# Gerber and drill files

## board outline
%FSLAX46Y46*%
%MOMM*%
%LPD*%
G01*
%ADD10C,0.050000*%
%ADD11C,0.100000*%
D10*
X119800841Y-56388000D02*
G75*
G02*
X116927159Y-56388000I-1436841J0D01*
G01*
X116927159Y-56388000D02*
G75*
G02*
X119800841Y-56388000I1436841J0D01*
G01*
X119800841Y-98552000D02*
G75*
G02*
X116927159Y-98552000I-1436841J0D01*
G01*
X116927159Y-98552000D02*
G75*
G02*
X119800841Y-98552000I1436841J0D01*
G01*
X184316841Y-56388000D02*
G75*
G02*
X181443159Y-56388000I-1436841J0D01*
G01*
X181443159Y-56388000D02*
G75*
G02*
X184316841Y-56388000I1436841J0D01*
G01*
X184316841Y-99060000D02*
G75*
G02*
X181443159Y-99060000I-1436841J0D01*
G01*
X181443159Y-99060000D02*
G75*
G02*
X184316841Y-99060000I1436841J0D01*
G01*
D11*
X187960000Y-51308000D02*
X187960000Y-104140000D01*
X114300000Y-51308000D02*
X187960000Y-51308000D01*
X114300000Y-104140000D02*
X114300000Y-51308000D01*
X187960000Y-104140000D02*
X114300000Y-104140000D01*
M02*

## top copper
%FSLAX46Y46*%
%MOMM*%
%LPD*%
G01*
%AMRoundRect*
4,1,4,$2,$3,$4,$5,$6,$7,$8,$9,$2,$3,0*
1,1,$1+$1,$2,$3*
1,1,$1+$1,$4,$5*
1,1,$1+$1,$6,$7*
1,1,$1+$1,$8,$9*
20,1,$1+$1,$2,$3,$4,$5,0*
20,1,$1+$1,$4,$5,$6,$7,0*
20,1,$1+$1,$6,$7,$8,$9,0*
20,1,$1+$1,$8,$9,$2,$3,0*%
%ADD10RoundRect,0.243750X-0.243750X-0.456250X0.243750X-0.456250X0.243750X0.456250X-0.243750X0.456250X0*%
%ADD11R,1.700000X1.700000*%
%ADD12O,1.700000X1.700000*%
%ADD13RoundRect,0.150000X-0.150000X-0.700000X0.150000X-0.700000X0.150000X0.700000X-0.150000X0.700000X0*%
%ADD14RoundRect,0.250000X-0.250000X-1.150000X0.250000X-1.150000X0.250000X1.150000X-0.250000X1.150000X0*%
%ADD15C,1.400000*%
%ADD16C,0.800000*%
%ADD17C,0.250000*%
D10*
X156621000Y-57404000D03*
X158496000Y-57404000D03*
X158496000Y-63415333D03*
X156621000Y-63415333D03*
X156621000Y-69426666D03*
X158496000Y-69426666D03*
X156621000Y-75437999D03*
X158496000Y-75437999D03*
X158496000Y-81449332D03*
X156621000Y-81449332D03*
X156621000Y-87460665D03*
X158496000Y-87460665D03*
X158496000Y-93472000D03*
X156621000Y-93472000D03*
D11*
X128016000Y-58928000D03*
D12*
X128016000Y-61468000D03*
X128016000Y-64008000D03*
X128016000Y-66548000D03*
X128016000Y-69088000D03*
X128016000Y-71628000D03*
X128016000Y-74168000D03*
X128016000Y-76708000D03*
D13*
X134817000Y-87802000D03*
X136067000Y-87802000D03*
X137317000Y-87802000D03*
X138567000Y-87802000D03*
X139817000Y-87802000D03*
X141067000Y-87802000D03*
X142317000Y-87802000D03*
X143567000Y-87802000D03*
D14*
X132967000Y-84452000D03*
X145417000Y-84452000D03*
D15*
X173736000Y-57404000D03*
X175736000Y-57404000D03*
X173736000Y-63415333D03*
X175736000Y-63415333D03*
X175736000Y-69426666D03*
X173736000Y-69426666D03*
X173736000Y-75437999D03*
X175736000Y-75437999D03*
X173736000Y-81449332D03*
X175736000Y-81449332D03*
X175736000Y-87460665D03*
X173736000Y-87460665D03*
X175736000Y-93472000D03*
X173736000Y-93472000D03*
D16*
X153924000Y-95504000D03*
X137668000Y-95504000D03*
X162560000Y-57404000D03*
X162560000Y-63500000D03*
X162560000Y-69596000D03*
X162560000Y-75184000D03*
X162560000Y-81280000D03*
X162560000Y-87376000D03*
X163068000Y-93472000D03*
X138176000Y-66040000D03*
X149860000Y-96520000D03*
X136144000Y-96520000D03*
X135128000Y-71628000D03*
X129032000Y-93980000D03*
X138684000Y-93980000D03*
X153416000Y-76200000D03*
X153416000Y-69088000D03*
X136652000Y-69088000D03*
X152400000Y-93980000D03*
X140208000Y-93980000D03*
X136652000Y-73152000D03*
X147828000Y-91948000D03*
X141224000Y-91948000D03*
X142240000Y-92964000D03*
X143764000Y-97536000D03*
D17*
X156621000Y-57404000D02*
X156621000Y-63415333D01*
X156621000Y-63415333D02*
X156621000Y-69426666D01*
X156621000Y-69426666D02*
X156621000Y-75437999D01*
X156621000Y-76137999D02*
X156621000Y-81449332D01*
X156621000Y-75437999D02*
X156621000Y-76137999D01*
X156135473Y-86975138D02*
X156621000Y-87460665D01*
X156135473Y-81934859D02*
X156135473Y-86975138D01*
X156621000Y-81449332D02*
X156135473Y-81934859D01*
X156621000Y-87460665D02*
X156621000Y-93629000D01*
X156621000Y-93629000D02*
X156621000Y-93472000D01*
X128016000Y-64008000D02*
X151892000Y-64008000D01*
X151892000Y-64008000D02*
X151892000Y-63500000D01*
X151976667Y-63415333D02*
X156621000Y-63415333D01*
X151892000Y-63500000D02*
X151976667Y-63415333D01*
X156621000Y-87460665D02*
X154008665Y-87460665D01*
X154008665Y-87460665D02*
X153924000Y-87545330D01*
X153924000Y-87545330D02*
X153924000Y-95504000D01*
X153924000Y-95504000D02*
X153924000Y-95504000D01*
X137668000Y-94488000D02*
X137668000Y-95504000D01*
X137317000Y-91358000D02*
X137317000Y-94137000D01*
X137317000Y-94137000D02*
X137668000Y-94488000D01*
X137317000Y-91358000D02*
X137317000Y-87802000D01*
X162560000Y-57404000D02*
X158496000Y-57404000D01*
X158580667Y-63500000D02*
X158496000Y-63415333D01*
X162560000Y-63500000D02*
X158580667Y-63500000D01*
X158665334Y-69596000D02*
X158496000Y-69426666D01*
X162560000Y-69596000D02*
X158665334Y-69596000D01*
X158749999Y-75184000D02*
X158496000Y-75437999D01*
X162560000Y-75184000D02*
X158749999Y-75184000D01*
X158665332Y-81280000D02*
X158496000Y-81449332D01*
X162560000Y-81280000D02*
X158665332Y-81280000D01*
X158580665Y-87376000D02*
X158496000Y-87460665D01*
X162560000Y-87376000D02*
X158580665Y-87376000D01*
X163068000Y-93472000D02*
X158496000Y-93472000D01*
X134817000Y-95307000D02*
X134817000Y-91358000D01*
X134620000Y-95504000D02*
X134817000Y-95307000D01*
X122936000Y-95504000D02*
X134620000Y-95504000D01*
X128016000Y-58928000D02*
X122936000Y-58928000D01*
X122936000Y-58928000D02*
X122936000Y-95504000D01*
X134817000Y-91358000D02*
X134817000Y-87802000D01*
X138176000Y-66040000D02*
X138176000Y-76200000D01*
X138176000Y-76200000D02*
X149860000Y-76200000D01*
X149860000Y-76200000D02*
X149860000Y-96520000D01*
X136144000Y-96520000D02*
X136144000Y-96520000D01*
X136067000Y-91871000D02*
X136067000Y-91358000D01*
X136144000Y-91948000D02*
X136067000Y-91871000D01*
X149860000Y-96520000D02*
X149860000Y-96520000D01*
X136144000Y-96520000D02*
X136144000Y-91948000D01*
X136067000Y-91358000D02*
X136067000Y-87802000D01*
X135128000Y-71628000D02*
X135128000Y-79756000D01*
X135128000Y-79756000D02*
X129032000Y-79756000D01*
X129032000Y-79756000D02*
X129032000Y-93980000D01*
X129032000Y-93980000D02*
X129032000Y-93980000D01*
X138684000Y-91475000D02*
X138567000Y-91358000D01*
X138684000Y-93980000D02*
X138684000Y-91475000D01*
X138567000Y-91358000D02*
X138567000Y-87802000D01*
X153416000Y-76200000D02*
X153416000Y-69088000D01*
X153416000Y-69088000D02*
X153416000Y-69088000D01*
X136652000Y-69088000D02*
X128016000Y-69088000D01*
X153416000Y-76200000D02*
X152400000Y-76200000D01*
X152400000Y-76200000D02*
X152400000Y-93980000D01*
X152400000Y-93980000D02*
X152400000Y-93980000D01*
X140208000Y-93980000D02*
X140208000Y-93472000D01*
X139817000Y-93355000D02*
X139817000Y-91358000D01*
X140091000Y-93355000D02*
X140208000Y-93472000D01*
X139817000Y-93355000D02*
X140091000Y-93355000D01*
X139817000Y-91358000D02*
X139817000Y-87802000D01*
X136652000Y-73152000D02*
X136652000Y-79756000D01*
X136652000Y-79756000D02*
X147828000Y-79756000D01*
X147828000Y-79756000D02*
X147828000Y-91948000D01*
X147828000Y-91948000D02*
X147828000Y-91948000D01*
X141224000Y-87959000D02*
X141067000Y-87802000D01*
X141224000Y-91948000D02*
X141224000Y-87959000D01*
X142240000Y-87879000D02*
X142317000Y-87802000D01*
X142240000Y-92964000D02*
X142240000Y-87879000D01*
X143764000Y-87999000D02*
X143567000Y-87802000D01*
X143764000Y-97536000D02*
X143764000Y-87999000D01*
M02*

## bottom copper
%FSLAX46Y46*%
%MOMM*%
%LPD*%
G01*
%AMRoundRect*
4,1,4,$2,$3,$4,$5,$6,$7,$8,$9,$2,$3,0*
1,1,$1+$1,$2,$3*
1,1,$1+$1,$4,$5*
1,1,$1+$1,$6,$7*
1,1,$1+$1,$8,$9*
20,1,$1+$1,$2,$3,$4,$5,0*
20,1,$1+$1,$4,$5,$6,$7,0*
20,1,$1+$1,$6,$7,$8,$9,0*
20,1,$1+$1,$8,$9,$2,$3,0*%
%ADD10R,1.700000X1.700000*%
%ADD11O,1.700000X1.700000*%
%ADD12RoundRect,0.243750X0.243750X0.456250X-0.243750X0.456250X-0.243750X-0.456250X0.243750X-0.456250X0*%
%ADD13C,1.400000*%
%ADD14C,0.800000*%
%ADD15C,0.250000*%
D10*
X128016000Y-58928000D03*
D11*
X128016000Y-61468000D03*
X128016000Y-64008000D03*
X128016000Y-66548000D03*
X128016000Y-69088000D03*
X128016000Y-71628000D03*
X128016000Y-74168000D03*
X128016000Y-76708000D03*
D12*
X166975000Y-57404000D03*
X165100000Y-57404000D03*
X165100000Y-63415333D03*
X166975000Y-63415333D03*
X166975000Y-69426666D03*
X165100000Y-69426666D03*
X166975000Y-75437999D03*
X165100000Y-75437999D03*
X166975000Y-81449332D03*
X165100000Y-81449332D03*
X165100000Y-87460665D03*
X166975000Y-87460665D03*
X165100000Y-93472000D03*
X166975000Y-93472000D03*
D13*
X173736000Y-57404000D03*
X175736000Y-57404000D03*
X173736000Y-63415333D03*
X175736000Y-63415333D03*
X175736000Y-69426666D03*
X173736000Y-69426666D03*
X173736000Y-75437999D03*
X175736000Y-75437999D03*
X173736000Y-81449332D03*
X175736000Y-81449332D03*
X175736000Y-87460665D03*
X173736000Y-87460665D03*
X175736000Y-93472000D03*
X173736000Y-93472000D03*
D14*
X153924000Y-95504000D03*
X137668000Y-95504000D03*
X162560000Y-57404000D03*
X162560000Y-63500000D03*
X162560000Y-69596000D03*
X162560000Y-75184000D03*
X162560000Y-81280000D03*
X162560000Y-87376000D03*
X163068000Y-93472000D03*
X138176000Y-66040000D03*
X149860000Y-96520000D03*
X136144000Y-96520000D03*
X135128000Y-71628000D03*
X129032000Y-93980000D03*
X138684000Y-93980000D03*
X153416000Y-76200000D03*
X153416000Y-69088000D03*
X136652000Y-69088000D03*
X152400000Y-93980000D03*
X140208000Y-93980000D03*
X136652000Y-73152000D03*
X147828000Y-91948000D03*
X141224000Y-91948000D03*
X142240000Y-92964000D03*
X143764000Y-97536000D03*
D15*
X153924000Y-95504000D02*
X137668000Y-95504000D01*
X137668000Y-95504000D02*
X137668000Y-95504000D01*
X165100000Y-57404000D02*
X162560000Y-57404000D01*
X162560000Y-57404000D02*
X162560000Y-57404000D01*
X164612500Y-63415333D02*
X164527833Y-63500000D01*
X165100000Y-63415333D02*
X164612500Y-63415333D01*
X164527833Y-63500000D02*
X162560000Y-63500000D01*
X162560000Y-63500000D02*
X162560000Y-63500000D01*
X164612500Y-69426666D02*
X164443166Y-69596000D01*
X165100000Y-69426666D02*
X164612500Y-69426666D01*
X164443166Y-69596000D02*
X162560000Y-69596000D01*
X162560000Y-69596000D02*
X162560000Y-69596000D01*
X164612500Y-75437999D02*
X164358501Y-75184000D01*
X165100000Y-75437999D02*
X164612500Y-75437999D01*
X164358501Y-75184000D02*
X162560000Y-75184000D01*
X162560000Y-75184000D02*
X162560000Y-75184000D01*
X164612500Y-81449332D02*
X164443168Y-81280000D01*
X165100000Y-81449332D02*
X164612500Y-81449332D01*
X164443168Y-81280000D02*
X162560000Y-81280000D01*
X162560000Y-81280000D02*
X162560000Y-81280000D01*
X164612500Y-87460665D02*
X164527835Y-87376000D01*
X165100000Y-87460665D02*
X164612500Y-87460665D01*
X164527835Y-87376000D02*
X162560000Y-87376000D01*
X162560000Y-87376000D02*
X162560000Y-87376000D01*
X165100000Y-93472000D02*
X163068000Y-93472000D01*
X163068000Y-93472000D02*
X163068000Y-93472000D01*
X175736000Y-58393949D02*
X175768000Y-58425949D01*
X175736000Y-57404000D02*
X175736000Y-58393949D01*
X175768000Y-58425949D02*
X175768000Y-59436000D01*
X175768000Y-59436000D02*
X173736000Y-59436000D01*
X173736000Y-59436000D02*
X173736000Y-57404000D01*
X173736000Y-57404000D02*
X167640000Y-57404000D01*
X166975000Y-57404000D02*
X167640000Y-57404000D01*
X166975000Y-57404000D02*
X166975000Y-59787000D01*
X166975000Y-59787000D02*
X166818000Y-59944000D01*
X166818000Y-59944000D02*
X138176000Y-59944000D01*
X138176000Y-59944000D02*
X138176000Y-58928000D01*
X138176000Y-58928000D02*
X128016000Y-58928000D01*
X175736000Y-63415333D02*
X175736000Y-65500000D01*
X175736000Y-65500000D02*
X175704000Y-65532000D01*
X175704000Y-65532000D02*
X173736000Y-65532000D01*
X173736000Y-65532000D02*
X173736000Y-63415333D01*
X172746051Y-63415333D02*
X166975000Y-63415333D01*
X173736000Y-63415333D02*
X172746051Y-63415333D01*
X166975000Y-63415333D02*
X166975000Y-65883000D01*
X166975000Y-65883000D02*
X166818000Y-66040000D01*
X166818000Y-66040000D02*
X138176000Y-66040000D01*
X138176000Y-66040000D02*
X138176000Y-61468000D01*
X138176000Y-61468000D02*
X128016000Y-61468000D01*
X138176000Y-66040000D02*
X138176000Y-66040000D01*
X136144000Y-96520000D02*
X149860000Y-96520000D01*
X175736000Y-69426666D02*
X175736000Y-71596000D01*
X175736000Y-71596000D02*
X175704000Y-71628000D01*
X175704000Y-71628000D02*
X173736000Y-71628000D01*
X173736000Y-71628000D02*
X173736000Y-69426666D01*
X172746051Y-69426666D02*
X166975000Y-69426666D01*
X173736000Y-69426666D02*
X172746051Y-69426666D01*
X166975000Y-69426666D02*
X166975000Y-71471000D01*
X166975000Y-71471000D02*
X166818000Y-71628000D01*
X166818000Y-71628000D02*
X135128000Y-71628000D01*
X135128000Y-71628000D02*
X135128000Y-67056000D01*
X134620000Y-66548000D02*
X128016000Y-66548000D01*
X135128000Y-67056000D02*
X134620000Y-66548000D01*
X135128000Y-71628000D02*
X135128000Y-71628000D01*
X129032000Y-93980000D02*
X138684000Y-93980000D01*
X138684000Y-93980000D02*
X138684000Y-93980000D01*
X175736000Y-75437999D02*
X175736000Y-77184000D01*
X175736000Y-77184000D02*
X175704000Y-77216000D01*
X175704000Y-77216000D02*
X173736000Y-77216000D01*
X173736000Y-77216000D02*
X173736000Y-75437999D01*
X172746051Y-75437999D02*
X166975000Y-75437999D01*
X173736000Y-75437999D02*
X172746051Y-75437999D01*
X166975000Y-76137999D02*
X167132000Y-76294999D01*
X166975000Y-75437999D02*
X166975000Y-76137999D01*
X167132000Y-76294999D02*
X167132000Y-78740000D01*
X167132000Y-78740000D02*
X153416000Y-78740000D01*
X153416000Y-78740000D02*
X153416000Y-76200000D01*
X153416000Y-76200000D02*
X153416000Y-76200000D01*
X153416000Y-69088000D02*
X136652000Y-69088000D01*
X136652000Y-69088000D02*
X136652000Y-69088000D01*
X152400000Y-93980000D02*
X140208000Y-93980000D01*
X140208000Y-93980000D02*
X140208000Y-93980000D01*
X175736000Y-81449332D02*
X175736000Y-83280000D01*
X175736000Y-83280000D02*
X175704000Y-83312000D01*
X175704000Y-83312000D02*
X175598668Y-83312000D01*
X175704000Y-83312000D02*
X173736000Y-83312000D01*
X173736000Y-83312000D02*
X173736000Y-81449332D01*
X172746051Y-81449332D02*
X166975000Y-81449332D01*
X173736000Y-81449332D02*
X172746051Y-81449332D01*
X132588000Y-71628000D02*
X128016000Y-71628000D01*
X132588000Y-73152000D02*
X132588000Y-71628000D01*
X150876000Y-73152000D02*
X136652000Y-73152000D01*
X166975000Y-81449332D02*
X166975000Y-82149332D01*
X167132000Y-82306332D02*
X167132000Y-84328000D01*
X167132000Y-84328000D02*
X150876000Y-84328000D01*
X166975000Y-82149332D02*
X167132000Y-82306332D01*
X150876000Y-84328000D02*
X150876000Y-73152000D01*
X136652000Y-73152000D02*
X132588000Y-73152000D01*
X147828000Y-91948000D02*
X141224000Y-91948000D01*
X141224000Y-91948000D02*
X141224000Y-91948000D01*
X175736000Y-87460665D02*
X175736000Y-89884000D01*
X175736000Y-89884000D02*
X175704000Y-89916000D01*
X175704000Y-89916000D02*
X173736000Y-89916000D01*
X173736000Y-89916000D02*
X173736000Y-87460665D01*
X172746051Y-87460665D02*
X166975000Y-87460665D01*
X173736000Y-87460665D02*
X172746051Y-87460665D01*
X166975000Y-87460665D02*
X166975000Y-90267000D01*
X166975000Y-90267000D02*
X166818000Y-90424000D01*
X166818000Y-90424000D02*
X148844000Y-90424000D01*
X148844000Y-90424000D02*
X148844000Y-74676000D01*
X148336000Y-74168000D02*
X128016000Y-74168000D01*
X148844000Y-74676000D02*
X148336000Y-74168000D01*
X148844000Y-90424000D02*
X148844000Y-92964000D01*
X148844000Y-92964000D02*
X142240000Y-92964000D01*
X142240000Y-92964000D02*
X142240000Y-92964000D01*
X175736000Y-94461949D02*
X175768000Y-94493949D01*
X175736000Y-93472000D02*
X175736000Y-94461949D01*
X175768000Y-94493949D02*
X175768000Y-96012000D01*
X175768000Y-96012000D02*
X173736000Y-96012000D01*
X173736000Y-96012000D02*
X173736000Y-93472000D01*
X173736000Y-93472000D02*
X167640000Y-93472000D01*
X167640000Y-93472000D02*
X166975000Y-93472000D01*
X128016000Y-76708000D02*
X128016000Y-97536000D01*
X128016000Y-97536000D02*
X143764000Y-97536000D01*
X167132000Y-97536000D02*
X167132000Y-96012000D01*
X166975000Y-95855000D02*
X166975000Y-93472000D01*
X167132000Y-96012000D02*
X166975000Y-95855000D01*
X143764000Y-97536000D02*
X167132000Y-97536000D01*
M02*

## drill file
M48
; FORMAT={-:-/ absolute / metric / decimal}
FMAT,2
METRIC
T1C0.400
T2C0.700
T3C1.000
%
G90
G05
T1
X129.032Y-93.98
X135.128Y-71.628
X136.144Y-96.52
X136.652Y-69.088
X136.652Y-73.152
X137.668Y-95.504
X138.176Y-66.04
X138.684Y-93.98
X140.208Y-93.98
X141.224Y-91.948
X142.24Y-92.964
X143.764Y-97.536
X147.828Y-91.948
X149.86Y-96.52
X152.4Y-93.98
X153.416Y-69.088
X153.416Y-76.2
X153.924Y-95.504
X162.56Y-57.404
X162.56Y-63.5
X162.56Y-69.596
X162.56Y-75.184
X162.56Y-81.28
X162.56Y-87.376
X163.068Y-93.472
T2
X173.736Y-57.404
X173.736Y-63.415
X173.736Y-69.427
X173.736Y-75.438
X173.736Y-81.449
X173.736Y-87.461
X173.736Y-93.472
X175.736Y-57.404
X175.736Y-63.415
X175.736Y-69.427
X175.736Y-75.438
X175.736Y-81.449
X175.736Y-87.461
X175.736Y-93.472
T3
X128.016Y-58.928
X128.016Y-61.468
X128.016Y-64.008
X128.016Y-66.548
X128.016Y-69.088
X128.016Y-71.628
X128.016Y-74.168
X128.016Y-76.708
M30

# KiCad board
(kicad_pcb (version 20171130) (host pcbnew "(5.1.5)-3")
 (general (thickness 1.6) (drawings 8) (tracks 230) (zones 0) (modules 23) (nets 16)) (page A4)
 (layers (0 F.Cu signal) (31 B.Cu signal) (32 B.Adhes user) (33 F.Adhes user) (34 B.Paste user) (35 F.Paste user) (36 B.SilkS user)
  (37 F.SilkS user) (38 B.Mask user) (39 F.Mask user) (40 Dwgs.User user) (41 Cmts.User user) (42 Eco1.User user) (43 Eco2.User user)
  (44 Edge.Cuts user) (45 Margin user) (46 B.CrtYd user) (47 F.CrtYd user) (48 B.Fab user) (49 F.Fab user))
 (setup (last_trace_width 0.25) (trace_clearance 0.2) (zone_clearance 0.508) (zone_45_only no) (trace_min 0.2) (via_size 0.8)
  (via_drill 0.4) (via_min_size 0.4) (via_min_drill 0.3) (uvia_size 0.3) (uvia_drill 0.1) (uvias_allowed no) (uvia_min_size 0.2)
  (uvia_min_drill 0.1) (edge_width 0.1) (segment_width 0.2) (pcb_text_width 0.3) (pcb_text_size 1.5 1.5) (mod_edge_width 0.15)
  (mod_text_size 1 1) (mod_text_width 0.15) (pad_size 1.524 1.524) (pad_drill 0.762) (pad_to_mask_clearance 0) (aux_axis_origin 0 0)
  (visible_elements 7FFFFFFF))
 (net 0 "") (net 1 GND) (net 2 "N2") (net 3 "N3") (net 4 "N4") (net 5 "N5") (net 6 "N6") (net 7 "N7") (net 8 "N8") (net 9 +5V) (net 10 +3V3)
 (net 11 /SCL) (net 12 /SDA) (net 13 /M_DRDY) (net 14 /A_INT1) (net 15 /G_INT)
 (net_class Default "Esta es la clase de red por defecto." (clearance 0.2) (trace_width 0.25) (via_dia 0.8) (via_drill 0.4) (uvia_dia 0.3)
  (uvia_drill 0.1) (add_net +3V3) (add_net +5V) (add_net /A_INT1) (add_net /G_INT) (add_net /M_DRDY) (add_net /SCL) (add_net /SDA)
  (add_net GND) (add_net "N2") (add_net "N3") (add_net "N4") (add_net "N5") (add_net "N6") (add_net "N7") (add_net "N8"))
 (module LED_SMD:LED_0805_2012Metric (layer F.Cu) (at 157.5585 57.404)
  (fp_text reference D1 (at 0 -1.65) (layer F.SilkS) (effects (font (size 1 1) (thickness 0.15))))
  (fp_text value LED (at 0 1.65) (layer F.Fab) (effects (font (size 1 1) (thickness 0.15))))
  (pad 1 smd roundrect (at -0.9375 0) (size 0.975 1.4) (layers F.Cu F.Paste F.Mask) (roundrect_rratio 0.25) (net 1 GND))
  (pad 2 smd roundrect (at 0.9375 0) (size 0.975 1.4) (layers F.Cu F.Paste F.Mask) (roundrect_rratio 0.25) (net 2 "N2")))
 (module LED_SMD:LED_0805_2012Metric (layer F.Cu) (at 157.5585 63.415333)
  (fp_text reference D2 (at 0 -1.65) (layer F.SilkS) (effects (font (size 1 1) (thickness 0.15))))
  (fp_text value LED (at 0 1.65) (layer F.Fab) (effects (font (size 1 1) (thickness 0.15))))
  (pad 2 smd roundrect (at 0.9375 0) (size 0.975 1.4) (layers F.Cu F.Paste F.Mask) (roundrect_rratio 0.25) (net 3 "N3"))
  (pad 1 smd roundrect (at -0.9375 0) (size 0.975 1.4) (layers F.Cu F.Paste F.Mask) (roundrect_rratio 0.25) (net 1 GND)))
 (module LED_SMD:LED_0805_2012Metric (layer F.Cu) (at 157.5585 69.426666)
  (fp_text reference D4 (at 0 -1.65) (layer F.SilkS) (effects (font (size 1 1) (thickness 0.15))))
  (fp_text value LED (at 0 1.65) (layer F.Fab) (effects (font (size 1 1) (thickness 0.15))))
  (pad 1 smd roundrect (at -0.9375 0) (size 0.975 1.4) (layers F.Cu F.Paste F.Mask) (roundrect_rratio 0.25) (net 1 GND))
  (pad 2 smd roundrect (at 0.9375 0) (size 0.975 1.4) (layers F.Cu F.Paste F.Mask) (roundrect_rratio 0.25) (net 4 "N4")))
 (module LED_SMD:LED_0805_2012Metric (layer F.Cu) (at 157.5585 75.437999)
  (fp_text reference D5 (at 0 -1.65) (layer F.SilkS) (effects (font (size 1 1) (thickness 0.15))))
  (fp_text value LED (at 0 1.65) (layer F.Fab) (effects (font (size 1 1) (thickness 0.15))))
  (pad 1 smd roundrect (at -0.9375 0) (size 0.975 1.4) (layers F.Cu F.Paste F.Mask) (roundrect_rratio 0.25) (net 1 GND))
  (pad 2 smd roundrect (at 0.9375 0) (size 0.975 1.4) (layers F.Cu F.Paste F.Mask) (roundrect_rratio 0.25) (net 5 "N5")))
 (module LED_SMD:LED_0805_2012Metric (layer F.Cu) (at 157.5585 81.449332)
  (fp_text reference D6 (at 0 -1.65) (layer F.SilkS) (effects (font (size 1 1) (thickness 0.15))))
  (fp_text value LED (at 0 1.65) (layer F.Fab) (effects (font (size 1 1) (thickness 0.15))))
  (pad 2 smd roundrect (at 0.9375 0) (size 0.975 1.4) (layers F.Cu F.Paste F.Mask) (roundrect_rratio 0.25) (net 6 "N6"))
  (pad 1 smd roundrect (at -0.9375 0) (size 0.975 1.4) (layers F.Cu F.Paste F.Mask) (roundrect_rratio 0.25) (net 1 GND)))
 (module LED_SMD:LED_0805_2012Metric (layer F.Cu) (at 157.5585 87.460665)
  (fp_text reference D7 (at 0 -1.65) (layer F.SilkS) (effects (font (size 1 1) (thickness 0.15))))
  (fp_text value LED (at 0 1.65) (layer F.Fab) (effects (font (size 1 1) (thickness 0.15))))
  (pad 1 smd roundrect (at -0.9375 0) (size 0.975 1.4) (layers F.Cu F.Paste F.Mask) (roundrect_rratio 0.25) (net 1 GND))
  (pad 2 smd roundrect (at 0.9375 0) (size 0.975 1.4) (layers F.Cu F.Paste F.Mask) (roundrect_rratio 0.25) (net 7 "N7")))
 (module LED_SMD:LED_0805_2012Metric (layer F.Cu) (at 157.5585 93.472)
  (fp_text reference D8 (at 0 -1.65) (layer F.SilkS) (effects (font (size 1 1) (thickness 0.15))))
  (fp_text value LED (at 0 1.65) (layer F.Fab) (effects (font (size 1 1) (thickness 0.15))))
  (pad 2 smd roundrect (at 0.9375 0) (size 0.975 1.4) (layers F.Cu F.Paste F.Mask) (roundrect_rratio 0.25) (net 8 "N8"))
  (pad 1 smd roundrect (at -0.9375 0) (size 0.975 1.4) (layers F.Cu F.Paste F.Mask) (roundrect_rratio 0.25) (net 1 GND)))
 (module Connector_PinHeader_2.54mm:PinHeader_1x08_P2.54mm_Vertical (layer F.Cu) (at 128.016 58.928)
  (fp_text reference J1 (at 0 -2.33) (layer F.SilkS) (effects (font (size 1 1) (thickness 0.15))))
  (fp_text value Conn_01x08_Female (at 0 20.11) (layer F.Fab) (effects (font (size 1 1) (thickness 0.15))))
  (pad 1 thru_hole rect (at 0 0) (size 1.7 1.7) (drill 1) (layers *.Cu *.Mask) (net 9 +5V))
  (pad 2 thru_hole oval (at 0 2.54) (size 1.7 1.7) (drill 1) (layers *.Cu *.Mask) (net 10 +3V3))
  (pad 3 thru_hole oval (at 0 5.08) (size 1.7 1.7) (drill 1) (layers *.Cu *.Mask) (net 1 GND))
  (pad 4 thru_hole oval (at 0 7.62) (size 1.7 1.7) (drill 1) (layers *.Cu *.Mask) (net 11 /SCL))
  (pad 5 thru_hole oval (at 0 10.16) (size 1.7 1.7) (drill 1) (layers *.Cu *.Mask) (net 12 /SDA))
  (pad 6 thru_hole oval (at 0 12.7) (size 1.7 1.7) (drill 1) (layers *.Cu *.Mask) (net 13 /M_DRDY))
  (pad 7 thru_hole oval (at 0 15.24) (size 1.7 1.7) (drill 1) (layers *.Cu *.Mask) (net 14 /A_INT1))
  (pad 8 thru_hole oval (at 0 17.78) (size 1.7 1.7) (drill 1) (layers *.Cu *.Mask) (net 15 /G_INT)))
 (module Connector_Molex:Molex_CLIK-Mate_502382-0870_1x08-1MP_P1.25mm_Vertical (layer F.Cu) (at 139.192 85.852)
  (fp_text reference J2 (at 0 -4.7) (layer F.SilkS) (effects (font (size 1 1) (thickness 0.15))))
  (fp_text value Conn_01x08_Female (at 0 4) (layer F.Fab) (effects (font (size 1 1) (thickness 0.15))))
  (pad 1 smd roundrect (at -4.375 1.95) (size 0.6 1.7) (layers F.Cu F.Paste F.Mask) (roundrect_rratio 0.25) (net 9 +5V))
  (pad 2 smd roundrect (at -3.125 1.95) (size 0.6 1.7) (layers F.Cu F.Paste F.Mask) (roundrect_rratio 0.25) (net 10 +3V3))
  (pad 3 smd roundrect (at -1.875 1.95) (size 0.6 1.7) (layers F.Cu F.Paste F.Mask) (roundrect_rratio 0.25) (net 1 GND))
  (pad 4 smd roundrect (at -0.625 1.95) (size 0.6 1.7) (layers F.Cu F.Paste F.Mask) (roundrect_rratio 0.25) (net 11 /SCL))
  (pad 5 smd roundrect (at 0.625 1.95) (size 0.6 1.7) (layers F.Cu F.Paste F.Mask) (roundrect_rratio 0.25) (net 12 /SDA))
  (pad 6 smd roundrect (at 1.875 1.95) (size 0.6 1.7) (layers F.Cu F.Paste F.Mask) (roundrect_rratio 0.25) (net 13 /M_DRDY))
  (pad 7 smd roundrect (at 3.125 1.95) (size 0.6 1.7) (layers F.Cu F.Paste F.Mask) (roundrect_rratio 0.25) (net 14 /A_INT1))
  (pad 8 smd roundrect (at 4.375 1.95) (size 0.6 1.7) (layers F.Cu F.Paste F.Mask) (roundrect_rratio 0.25) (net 15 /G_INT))
  (pad MP smd roundrect (at -6.225 -1.4) (size 1 2.8) (layers F.Cu F.Paste F.Mask) (roundrect_rratio 0.25))
  (pad MP smd roundrect (at 6.225 -1.4) (size 1 2.8) (layers F.Cu F.Paste F.Mask) (roundrect_rratio 0.25)))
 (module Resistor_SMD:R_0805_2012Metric (layer B.Cu) (at 166.0375 57.404 180)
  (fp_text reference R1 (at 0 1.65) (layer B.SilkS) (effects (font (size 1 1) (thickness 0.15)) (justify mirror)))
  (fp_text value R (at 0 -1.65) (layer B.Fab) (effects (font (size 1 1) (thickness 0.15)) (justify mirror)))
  (pad 1 smd roundrect (at -0.9375 0 180) (size 0.975 1.4) (layers B.Cu B.Paste B.Mask) (roundrect_rratio 0.25) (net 9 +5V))
  (pad 2 smd roundrect (at 0.9375 0 180) (size 0.975 1.4) (layers B.Cu B.Paste B.Mask) (roundrect_rratio 0.25) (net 2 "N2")))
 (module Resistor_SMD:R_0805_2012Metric (layer B.Cu) (at 166.0375 63.415333 180)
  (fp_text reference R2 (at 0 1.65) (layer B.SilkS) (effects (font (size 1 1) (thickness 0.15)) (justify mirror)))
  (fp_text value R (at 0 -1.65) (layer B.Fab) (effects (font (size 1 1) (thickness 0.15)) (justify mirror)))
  (pad 2 smd roundrect (at 0.9375 0 180) (size 0.975 1.4) (layers B.Cu B.Paste B.Mask) (roundrect_rratio 0.25) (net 3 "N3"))
  (pad 1 smd roundrect (at -0.9375 0 180) (size 0.975 1.4) (layers B.Cu B.Paste B.Mask) (roundrect_rratio 0.25) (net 10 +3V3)))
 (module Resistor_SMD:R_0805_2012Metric (layer B.Cu) (at 166.0375 69.426666 180)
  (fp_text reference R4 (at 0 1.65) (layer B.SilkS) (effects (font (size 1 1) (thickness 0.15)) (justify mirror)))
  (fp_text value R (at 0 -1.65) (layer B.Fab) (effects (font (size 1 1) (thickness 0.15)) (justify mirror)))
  (pad 1 smd roundrect (at -0.9375 0 180) (size 0.975 1.4) (layers B.Cu B.Paste B.Mask) (roundrect_rratio 0.25) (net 11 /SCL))
  (pad 2 smd roundrect (at 0.9375 0 180) (size 0.975 1.4) (layers B.Cu B.Paste B.Mask) (roundrect_rratio 0.25) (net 4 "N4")))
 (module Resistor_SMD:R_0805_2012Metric (layer B.Cu) (at 166.0375 75.437999 180)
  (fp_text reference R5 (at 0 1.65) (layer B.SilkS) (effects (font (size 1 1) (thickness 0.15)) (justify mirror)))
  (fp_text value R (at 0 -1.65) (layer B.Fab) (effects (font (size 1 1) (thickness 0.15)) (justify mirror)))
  (pad 1 smd roundrect (at -0.9375 0 180) (size 0.975 1.4) (layers B.Cu B.Paste B.Mask) (roundrect_rratio 0.25) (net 12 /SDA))
  (pad 2 smd roundrect (at 0.9375 0 180) (size 0.975 1.4) (layers B.Cu B.Paste B.Mask) (roundrect_rratio 0.25) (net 5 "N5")))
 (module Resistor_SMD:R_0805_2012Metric (layer B.Cu) (at 166.0375 81.449332 180)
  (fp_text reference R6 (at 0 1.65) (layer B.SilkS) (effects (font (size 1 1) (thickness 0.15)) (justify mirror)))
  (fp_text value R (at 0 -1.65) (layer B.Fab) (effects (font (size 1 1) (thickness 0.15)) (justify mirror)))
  (pad 1 smd roundrect (at -0.9375 0 180) (size 0.975 1.4) (layers B.Cu B.Paste B.Mask) (roundrect_rratio 0.25) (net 13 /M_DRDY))
  (pad 2 smd roundrect (at 0.9375 0 180) (size 0.975 1.4) (layers B.Cu B.Paste B.Mask) (roundrect_rratio 0.25) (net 6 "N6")))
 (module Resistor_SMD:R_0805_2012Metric (layer B.Cu) (at 166.0375 87.460665 180)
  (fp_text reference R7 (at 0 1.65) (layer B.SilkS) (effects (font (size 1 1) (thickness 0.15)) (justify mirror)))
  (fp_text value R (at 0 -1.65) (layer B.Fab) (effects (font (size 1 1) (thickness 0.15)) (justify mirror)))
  (pad 2 smd roundrect (at 0.9375 0 180) (size 0.975 1.4) (layers B.Cu B.Paste B.Mask) (roundrect_rratio 0.25) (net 7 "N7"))
  (pad 1 smd roundrect (at -0.9375 0 180) (size 0.975 1.4) (layers B.Cu B.Paste B.Mask) (roundrect_rratio 0.25) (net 14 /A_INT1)))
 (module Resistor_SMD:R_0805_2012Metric (layer B.Cu) (at 166.0375 93.472 180)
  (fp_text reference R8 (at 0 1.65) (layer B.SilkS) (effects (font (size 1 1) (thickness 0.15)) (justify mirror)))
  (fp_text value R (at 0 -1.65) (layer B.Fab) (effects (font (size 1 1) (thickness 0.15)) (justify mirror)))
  (pad 2 smd roundrect (at 0.9375 0 180) (size 0.975 1.4) (layers B.Cu B.Paste B.Mask) (roundrect_rratio 0.25) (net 8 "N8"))
  (pad 1 smd roundrect (at -0.9375 0 180) (size 0.975 1.4) (layers B.Cu B.Paste B.Mask) (roundrect_rratio 0.25) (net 15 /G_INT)))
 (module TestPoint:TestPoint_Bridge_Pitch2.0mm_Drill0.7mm (layer F.Cu) (at 173.736 57.404)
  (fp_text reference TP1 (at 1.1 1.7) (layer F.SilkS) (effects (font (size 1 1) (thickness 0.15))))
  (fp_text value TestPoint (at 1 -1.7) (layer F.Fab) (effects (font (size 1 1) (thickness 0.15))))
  (pad 1 thru_hole circle (at 0 0) (size 1.4 1.4) (drill 0.7) (layers *.Cu *.Mask) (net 9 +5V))
  (pad 1 thru_hole circle (at 2 0) (size 1.4 1.4) (drill 0.7) (layers *.Cu *.Mask) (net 9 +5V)))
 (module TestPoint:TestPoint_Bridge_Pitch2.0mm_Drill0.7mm (layer F.Cu) (at 173.736 63.415333)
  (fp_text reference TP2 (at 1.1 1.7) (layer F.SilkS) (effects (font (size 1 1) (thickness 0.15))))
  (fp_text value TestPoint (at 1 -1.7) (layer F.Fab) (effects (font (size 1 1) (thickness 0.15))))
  (pad 1 thru_hole circle (at 0 0) (size 1.4 1.4) (drill 0.7) (layers *.Cu *.Mask) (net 10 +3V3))
  (pad 1 thru_hole circle (at 2 0) (size 1.4 1.4) (drill 0.7) (layers *.Cu *.Mask) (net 10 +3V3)))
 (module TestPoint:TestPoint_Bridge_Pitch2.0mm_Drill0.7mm (layer F.Cu) (at 173.736 69.426666)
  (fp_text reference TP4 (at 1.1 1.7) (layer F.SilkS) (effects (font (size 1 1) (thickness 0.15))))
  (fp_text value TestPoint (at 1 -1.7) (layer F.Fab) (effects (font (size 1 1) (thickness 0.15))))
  (pad 1 thru_hole circle (at 2 0) (size 1.4 1.4) (drill 0.7) (layers *.Cu *.Mask) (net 11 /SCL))
  (pad 1 thru_hole circle (at 0 0) (size 1.4 1.4) (drill 0.7) (layers *.Cu *.Mask) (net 11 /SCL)))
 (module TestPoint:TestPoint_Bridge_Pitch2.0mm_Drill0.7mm (layer F.Cu) (at 173.736 75.437999)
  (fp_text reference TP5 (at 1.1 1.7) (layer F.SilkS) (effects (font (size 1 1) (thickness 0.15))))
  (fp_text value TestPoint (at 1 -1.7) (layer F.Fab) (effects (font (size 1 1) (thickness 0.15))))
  (pad 1 thru_hole circle (at 0 0) (size 1.4 1.4) (drill 0.7) (layers *.Cu *.Mask) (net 12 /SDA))
  (pad 1 thru_hole circle (at 2 0) (size 1.4 1.4) (drill 0.7) (layers *.Cu *.Mask) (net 12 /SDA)))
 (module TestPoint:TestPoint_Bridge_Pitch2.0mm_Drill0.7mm (layer F.Cu) (at 173.736 81.449332)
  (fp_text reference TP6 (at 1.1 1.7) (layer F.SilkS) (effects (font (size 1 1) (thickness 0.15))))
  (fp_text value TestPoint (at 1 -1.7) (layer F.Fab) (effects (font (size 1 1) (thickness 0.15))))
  (pad 1 thru_hole circle (at 0 0) (size 1.4 1.4) (drill 0.7) (layers *.Cu *.Mask) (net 13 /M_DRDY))
  (pad 1 thru_hole circle (at 2 0) (size 1.4 1.4) (drill 0.7) (layers *.Cu *.Mask) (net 13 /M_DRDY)))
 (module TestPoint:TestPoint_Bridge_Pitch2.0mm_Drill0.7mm (layer F.Cu) (at 173.736 87.460665)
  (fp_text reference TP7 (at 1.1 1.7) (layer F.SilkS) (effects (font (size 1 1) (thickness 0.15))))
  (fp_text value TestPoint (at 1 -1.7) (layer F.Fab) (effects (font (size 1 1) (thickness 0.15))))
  (pad 1 thru_hole circle (at 2 0) (size 1.4 1.4) (drill 0.7) (layers *.Cu *.Mask) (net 14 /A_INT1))
  (pad 1 thru_hole circle (at 0 0) (size 1.4 1.4) (drill 0.7) (layers *.Cu *.Mask) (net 14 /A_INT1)))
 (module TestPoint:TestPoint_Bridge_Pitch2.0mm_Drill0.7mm (layer F.Cu) (at 173.736 93.472)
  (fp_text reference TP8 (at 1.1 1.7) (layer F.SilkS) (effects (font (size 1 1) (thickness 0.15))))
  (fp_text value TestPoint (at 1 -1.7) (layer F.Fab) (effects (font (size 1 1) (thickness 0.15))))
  (pad 1 thru_hole circle (at 2 0) (size 1.4 1.4) (drill 0.7) (layers *.Cu *.Mask) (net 15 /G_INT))
  (pad 1 thru_hole circle (at 0 0) (size 1.4 1.4) (drill 0.7) (layers *.Cu *.Mask) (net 15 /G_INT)))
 (gr_circle (center 118.364 56.388) (end 119.38 57.404) (layer Edge.Cuts) (width 0.05))
 (gr_circle (center 118.364 98.552) (end 119.38 99.568) (layer Edge.Cuts) (width 0.05))
 (gr_circle (center 182.88 56.388) (end 183.896 57.404) (layer Edge.Cuts) (width 0.05))
 (gr_circle (center 182.88 99.06) (end 183.896 100.076) (layer Edge.Cuts) (width 0.05))
 (gr_line (start 187.96 51.308) (end 187.96 104.14) (layer Edge.Cuts) (width 0.1))
 (gr_line (start 114.3 51.308) (end 187.96 51.308) (layer Edge.Cuts) (width 0.1))
 (gr_line (start 114.3 104.14) (end 114.3 51.308) (layer Edge.Cuts) (width 0.1))
 (gr_line (start 187.96 104.14) (end 114.3 104.14) (layer Edge.Cuts) (width 0.1))
 (segment (start 156.621 57.404) (end 156.621 63.415333) (width 0.25) (layer F.Cu) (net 1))
 (segment (start 156.621 63.415333) (end 156.621 69.426666) (width 0.25) (layer F.Cu) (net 1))
 (segment (start 156.621 69.426666) (end 156.621 75.437999) (width 0.25) (layer F.Cu) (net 1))
 (segment (start 156.621 76.137999) (end 156.621 81.449332) (width 0.25) (layer F.Cu) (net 1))
 (segment (start 156.621 75.437999) (end 156.621 76.137999) (width 0.25) (layer F.Cu) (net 1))
 (segment (start 156.135473 86.975138) (end 156.621 87.460665) (width 0.25) (layer F.Cu) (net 1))
 (segment (start 156.135473 81.934859) (end 156.135473 86.975138) (width 0.25) (layer F.Cu) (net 1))
 (segment (start 156.621 81.449332) (end 156.135473 81.934859) (width 0.25) (layer F.Cu) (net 1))
 (segment (start 156.621 87.460665) (end 156.621 93.629) (width 0.25) (layer F.Cu) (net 1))
 (segment (start 156.621 93.629) (end 156.621 93.472) (width 0.25) (layer F.Cu) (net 1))
 (segment (start 128.016 64.008) (end 151.892 64.008) (width 0.25) (layer F.Cu) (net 1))
 (segment (start 151.892 64.008) (end 151.892 63.5) (width 0.25) (layer F.Cu) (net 1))
 (segment (start 151.976667 63.415333) (end 156.621 63.415333) (width 0.25) (layer F.Cu) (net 1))
 (segment (start 151.892 63.5) (end 151.976667 63.415333) (width 0.25) (layer F.Cu) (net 1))
 (segment (start 156.621 87.460665) (end 154.008665 87.460665) (width 0.25) (layer F.Cu) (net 1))
 (segment (start 154.008665 87.460665) (end 153.924 87.54533) (width 0.25) (layer F.Cu) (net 1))
 (segment (start 153.924 87.54533) (end 153.924 95.504) (width 0.25) (layer F.Cu) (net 1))
 (segment (start 153.924 95.504) (end 153.924 95.504) (width 0.25) (layer F.Cu) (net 1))
 (via (at 153.924 95.504) (size 0.8) (drill 0.4) (layers F.Cu B.Cu) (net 1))
 (segment (start 153.924 95.504) (end 137.668 95.504) (width 0.25) (layer B.Cu) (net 1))
 (segment (start 137.668 95.504) (end 137.668 95.504) (width 0.25) (layer B.Cu) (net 1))
 (via (at 137.668 95.504) (size 0.8) (drill 0.4) (layers F.Cu B.Cu) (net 1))
 (segment (start 137.668 94.488) (end 137.668 95.504) (width 0.25) (layer F.Cu) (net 1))
 (segment (start 137.317 91.358) (end 137.317 94.137) (width 0.25) (layer F.Cu) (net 1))
 (segment (start 137.317 94.137) (end 137.668 94.488) (width 0.25) (layer F.Cu) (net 1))
 (segment (start 137.317 91.358) (end 137.317 87.802) (width 0.25) (layer F.Cu) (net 1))
 (segment (start 165.1 57.404) (end 162.56 57.404) (width 0.25) (layer B.Cu) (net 2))
 (segment (start 162.56 57.404) (end 162.56 57.404) (width 0.25) (layer B.Cu) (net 2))
 (via (at 162.56 57.404) (size 0.8) (drill 0.4) (layers F.Cu B.Cu) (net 2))
 (segment (start 162.56 57.404) (end 158.496 57.404) (width 0.25) (layer F.Cu) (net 2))
 (segment (start 164.6125 63.415333) (end 164.527833 63.5) (width 0.25) (layer B.Cu) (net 3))
 (segment (start 165.1 63.415333) (end 164.6125 63.415333) (width 0.25) (layer B.Cu) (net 3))
 (segment (start 164.527833 63.5) (end 162.56 63.5) (width 0.25) (layer B.Cu) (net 3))
 (segment (start 162.56 63.5) (end 162.56 63.5) (width 0.25) (layer B.Cu) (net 3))
 (via (at 162.56 63.5) (size 0.8) (drill 0.4) (layers F.Cu B.Cu) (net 3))
 (segment (start 158.580667 63.5) (end 158.496 63.415333) (width 0.25) (layer F.Cu) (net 3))
 (segment (start 162.56 63.5) (end 158.580667 63.5) (width 0.25) (layer F.Cu) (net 3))
 (segment (start 164.6125 69.426666) (end 164.443166 69.596) (width 0.25) (layer B.Cu) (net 4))
 (segment (start 165.1 69.426666) (end 164.6125 69.426666) (width 0.25) (layer B.Cu) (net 4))
 (segment (start 164.443166 69.596) (end 162.56 69.596) (width 0.25) (layer B.Cu) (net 4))
 (segment (start 162.56 69.596) (end 162.56 69.596) (width 0.25) (layer B.Cu) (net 4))
 (via (at 162.56 69.596) (size 0.8) (drill 0.4) (layers F.Cu B.Cu) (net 4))
 (segment (start 158.665334 69.596) (end 158.496 69.426666) (width 0.25) (layer F.Cu) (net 4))
 (segment (start 162.56 69.596) (end 158.665334 69.596) (width 0.25) (layer F.Cu) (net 4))
 (segment (start 164.6125 75.437999) (end 164.358501 75.184) (width 0.25) (layer B.Cu) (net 5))
 (segment (start 165.1 75.437999) (end 164.6125 75.437999) (width 0.25) (layer B.Cu) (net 5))
 (segment (start 164.358501 75.184) (end 162.56 75.184) (width 0.25) (layer B.Cu) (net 5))
 (segment (start 162.56 75.184) (end 162.56 75.184) (width 0.25) (layer B.Cu) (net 5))
 (via (at 162.56 75.184) (size 0.8) (drill 0.4) (layers F.Cu B.Cu) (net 5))
 (segment (start 158.749999 75.184) (end 158.496 75.437999) (width 0.25) (layer F.Cu) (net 5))
 (segment (start 162.56 75.184) (end 158.749999 75.184) (width 0.25) (layer F.Cu) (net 5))
 (segment (start 164.6125 81.449332) (end 164.443168 81.28) (width 0.25) (layer B.Cu) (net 6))
 (segment (start 165.1 81.449332) (end 164.6125 81.449332) (width 0.25) (layer B.Cu) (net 6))
 (segment (start 164.443168 81.28) (end 162.56 81.28) (width 0.25) (layer B.Cu) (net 6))
 (segment (start 162.56 81.28) (end 162.56 81.28) (width 0.25) (layer B.Cu) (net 6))
 (via (at 162.56 81.28) (size 0.8) (drill 0.4) (layers F.Cu B.Cu) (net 6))
 (segment (start 158.665332 81.28) (end 158.496 81.449332) (width 0.25) (layer F.Cu) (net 6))
 (segment (start 162.56 81.28) (end 158.665332 81.28) (width 0.25) (layer F.Cu) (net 6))
 (segment (start 164.6125 87.460665) (end 164.527835 87.376) (width 0.25) (layer B.Cu) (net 7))
 (segment (start 165.1 87.460665) (end 164.6125 87.460665) (width 0.25) (layer B.Cu) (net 7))
 (segment (start 164.527835 87.376) (end 162.56 87.376) (width 0.25) (layer B.Cu) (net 7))
 (segment (start 162.56 87.376) (end 162.56 87.376) (width 0.25) (layer B.Cu) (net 7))
 (via (at 162.56 87.376) (size 0.8) (drill 0.4) (layers F.Cu B.Cu) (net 7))
 (segment (start 158.580665 87.376) (end 158.496 87.460665) (width 0.25) (layer F.Cu) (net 7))
 (segment (start 162.56 87.376) (end 158.580665 87.376) (width 0.25) (layer F.Cu) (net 7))
 (segment (start 165.1 93.472) (end 163.068 93.472) (width 0.25) (layer B.Cu) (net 8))
 (segment (start 163.068 93.472) (end 163.068 93.472) (width 0.25) (layer B.Cu) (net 8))
 (via (at 163.068 93.472) (size 0.8) (drill 0.4) (layers F.Cu B.Cu) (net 8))
 (segment (start 163.068 93.472) (end 158.496 93.472) (width 0.25) (layer F.Cu) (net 8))
 (segment (start 175.736 58.393949) (end 175.768 58.425949) (width 0.25) (layer B.Cu) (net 9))
 (segment (start 175.736 57.404) (end 175.736 58.393949) (width 0.25) (layer B.Cu) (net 9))
 (segment (start 175.768 58.425949) (end 175.768 59.436) (width 0.25) (layer B.Cu) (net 9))
 (segment (start 175.768 59.436) (end 173.736 59.436) (width 0.25) (layer B.Cu) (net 9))
 (segment (start 173.736 59.436) (end 173.736 57.404) (width 0.25) (layer B.Cu) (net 9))
 (segment (start 173.736 57.404) (end 167.64 57.404) (width 0.25) (layer B.Cu) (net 9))
 (segment (start 166.975 57.404) (end 167.64 57.404) (width 0.25) (layer B.Cu) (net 9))
 (segment (start 166.975 57.404) (end 166.975 59.787) (width 0.25) (layer B.Cu) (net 9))
 (segment (start 166.975 59.787) (end 166.818 59.944) (width 0.25) (layer B.Cu) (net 9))
 (segment (start 166.818 59.944) (end 138.176 59.944) (width 0.25) (layer B.Cu) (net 9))
 (segment (start 138.176 59.944) (end 138.176 58.928) (width 0.25) (layer B.Cu) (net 9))
 (segment (start 138.176 58.928) (end 128.016 58.928) (width 0.25) (layer B.Cu) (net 9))
 (segment (start 134.817 95.307) (end 134.817 91.358) (width 0.25) (layer F.Cu) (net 9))
 (segment (start 134.62 95.504) (end 134.817 95.307) (width 0.25) (layer F.Cu) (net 9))
 (segment (start 122.936 95.504) (end 134.62 95.504) (width 0.25) (layer F.Cu) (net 9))
 (segment (start 128.016 58.928) (end 122.936 58.928) (width 0.25) (layer F.Cu) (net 9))
 (segment (start 122.936 58.928) (end 122.936 95.504) (width 0.25) (layer F.Cu) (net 9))
 (segment (start 134.817 91.358) (end 134.817 87.802) (width 0.25) (layer F.Cu) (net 9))
 (segment (start 175.736 63.415333) (end 175.736 65.5) (width 0.25) (layer B.Cu) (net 10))
 (segment (start 175.736 65.5) (end 175.704 65.532) (width 0.25) (layer B.Cu) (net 10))
 (segment (start 175.704 65.532) (end 173.736 65.532) (width 0.25) (layer B.Cu) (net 10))
 (segment (start 173.736 65.532) (end 173.736 63.415333) (width 0.25) (layer B.Cu) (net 10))
 (segment (start 172.746051 63.415333) (end 166.975 63.415333) (width 0.25) (layer B.Cu) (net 10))
 (segment (start 173.736 63.415333) (end 172.746051 63.415333) (width 0.25) (layer B.Cu) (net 10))
 (segment (start 166.975 63.415333) (end 166.975 65.883) (width 0.25) (layer B.Cu) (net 10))
 (segment (start 166.975 65.883) (end 166.818 66.04) (width 0.25) (layer B.Cu) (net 10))
 (segment (start 166.818 66.04) (end 138.176 66.04) (width 0.25) (layer B.Cu) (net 10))
 (segment (start 138.176 66.04) (end 138.176 61.468) (width 0.25) (layer B.Cu) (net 10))
 (segment (start 138.176 61.468) (end 128.016 61.468) (width 0.25) (layer B.Cu) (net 10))
 (segment (start 138.176 66.04) (end 138.176 66.04) (width 0.25) (layer B.Cu) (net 10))
 (via (at 138.176 66.04) (size 0.8) (drill 0.4) (layers F.Cu B.Cu) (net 10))
 (segment (start 138.176 66.04) (end 138.176 76.2) (width 0.25) (layer F.Cu) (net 10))
 (segment (start 138.176 76.2) (end 149.86 76.2) (width 0.25) (layer F.Cu) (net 10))
 (segment (start 149.86 76.2) (end 149.86 96.52) (width 0.25) (layer F.Cu) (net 10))
 (segment (start 136.144 96.52) (end 136.144 96.52) (width 0.25) (layer F.Cu) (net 10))
 (segment (start 136.067 91.871) (end 136.067 91.358) (width 0.25) (layer F.Cu) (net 10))
 (segment (start 136.144 91.948) (end 136.067 91.871) (width 0.25) (layer F.Cu) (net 10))
 (segment (start 149.86 96.52) (end 149.86 96.52) (width 0.25) (layer F.Cu) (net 10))
 (via (at 149.86 96.52) (size 0.8) (drill 0.4) (layers F.Cu B.Cu) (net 10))
 (segment (start 136.144 96.52) (end 136.144 91.948) (width 0.25) (layer F.Cu) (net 10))
 (via (at 136.144 96.52) (size 0.8) (drill 0.4) (layers F.Cu B.Cu) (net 10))
 (segment (start 136.144 96.52) (end 149.86 96.52) (width 0.25) (layer B.Cu) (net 10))
 (segment (start 136.067 91.358) (end 136.067 87.802) (width 0.25) (layer F.Cu) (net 10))
 (segment (start 175.736 69.426666) (end 175.736 71.596) (width 0.25) (layer B.Cu) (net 11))
 (segment (start 175.736 71.596) (end 175.704 71.628) (width 0.25) (layer B.Cu) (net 11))
 (segment (start 175.704 71.628) (end 173.736 71.628) (width 0.25) (layer B.Cu) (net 11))
 (segment (start 173.736 71.628) (end 173.736 69.426666) (width 0.25) (layer B.Cu) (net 11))
 (segment (start 172.746051 69.426666) (end 166.975 69.426666) (width 0.25) (layer B.Cu) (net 11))
 (segment (start 173.736 69.426666) (end 172.746051 69.426666) (width 0.25) (layer B.Cu) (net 11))
 (segment (start 166.975 69.426666) (end 166.975 71.471) (width 0.25) (layer B.Cu) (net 11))
 (segment (start 166.975 71.471) (end 166.818 71.628) (width 0.25) (layer B.Cu) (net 11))
 (segment (start 166.818 71.628) (end 135.128 71.628) (width 0.25) (layer B.Cu) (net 11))
 (segment (start 135.128 71.628) (end 135.128 67.056) (width 0.25) (layer B.Cu) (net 11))
 (segment (start 134.62 66.548) (end 128.016 66.548) (width 0.25) (layer B.Cu) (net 11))
 (segment (start 135.128 67.056) (end 134.62 66.548) (width 0.25) (layer B.Cu) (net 11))
 (segment (start 135.128 71.628) (end 135.128 71.628) (width 0.25) (layer B.Cu) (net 11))
 (via (at 135.128 71.628) (size 0.8) (drill 0.4) (layers F.Cu B.Cu) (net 11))
 (segment (start 135.128 71.628) (end 135.128 79.756) (width 0.25) (layer F.Cu) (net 11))
 (segment (start 135.128 79.756) (end 129.032 79.756) (width 0.25) (layer F.Cu) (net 11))
 (segment (start 129.032 79.756) (end 129.032 93.98) (width 0.25) (layer F.Cu) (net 11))
 (segment (start 129.032 93.98) (end 129.032 93.98) (width 0.25) (layer F.Cu) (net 11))
 (via (at 129.032 93.98) (size 0.8) (drill 0.4) (layers F.Cu B.Cu) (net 11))
 (segment (start 129.032 93.98) (end 138.684 93.98) (width 0.25) (layer B.Cu) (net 11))
 (segment (start 138.684 93.98) (end 138.684 93.98) (width 0.25) (layer B.Cu) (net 11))
 (via (at 138.684 93.98) (size 0.8) (drill 0.4) (layers F.Cu B.Cu) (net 11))
 (segment (start 138.684 91.475) (end 138.567 91.358) (width 0.25) (layer F.Cu) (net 11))
 (segment (start 138.684 93.98) (end 138.684 91.475) (width 0.25) (layer F.Cu) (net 11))
 (segment (start 138.567 91.358) (end 138.567 87.802) (width 0.25) (layer F.Cu) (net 11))
 (segment (start 175.736 75.437999) (end 175.736 77.184) (width 0.25) (layer B.Cu) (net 12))
 (segment (start 175.736 77.184) (end 175.704 77.216) (width 0.25) (layer B.Cu) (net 12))
 (segment (start 175.704 77.216) (end 173.736 77.216) (width 0.25) (layer B.Cu) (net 12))
 (segment (start 173.736 77.216) (end 173.736 75.437999) (width 0.25) (layer B.Cu) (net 12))
 (segment (start 172.746051 75.437999) (end 166.975 75.437999) (width 0.25) (layer B.Cu) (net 12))
 (segment (start 173.736 75.437999) (end 172.746051 75.437999) (width 0.25) (layer B.Cu) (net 12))
 (segment (start 166.975 76.137999) (end 167.132 76.294999) (width 0.25) (layer B.Cu) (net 12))
 (segment (start 166.975 75.437999) (end 166.975 76.137999) (width 0.25) (layer B.Cu) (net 12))
 (segment (start 167.132 76.294999) (end 167.132 78.74) (width 0.25) (layer B.Cu) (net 12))
 (segment (start 167.132 78.74) (end 153.416 78.74) (width 0.25) (layer B.Cu) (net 12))
 (segment (start 153.416 78.74) (end 153.416 76.2) (width 0.25) (layer B.Cu) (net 12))
 (segment (start 153.416 76.2) (end 153.416 76.2) (width 0.25) (layer B.Cu) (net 12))
 (via (at 153.416 76.2) (size 0.8) (drill 0.4) (layers F.Cu B.Cu) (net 12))
 (segment (start 153.416 76.2) (end 153.416 69.088) (width 0.25) (layer F.Cu) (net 12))
 (segment (start 153.416 69.088) (end 153.416 69.088) (width 0.25) (layer F.Cu) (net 12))
 (via (at 153.416 69.088) (size 0.8) (drill 0.4) (layers F.Cu B.Cu) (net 12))
 (segment (start 153.416 69.088) (end 136.652 69.088) (width 0.25) (layer B.Cu) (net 12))
 (segment (start 136.652 69.088) (end 136.652 69.088) (width 0.25) (layer B.Cu) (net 12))
 (via (at 136.652 69.088) (size 0.8) (drill 0.4) (layers F.Cu B.Cu) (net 12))
 (segment (start 136.652 69.088) (end 128.016 69.088) (width 0.25) (layer F.Cu) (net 12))
 (segment (start 153.416 76.2) (end 152.4 76.2) (width 0.25) (layer F.Cu) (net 12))
 (segment (start 152.4 76.2) (end 152.4 93.98) (width 0.25) (layer F.Cu) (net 12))
 (segment (start 152.4 93.98) (end 152.4 93.98) (width 0.25) (layer F.Cu) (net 12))
 (via (at 152.4 93.98) (size 0.8) (drill 0.4) (layers F.Cu B.Cu) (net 12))
 (segment (start 152.4 93.98) (end 140.208 93.98) (width 0.25) (layer B.Cu) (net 12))
 (segment (start 140.208 93.98) (end 140.208 93.98) (width 0.25) (layer B.Cu) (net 12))
 (via (at 140.208 93.98) (size 0.8) (drill 0.4) (layers F.Cu B.Cu) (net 12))
 (segment (start 140.208 93.98) (end 140.208 93.472) (width 0.25) (layer F.Cu) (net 12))
 (segment (start 139.817 93.355) (end 139.817 91.358) (width 0.25) (layer F.Cu) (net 12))
 (segment (start 140.091 93.355) (end 140.208 93.472) (width 0.25) (layer F.Cu) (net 12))
 (segment (start 139.817 93.355) (end 140.091 93.355) (width 0.25) (layer F.Cu) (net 12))
 (segment (start 139.817 91.358) (end 139.817 87.802) (width 0.25) (layer F.Cu) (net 12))
 (segment (start 175.736 81.449332) (end 175.736 83.28) (width 0.25) (layer B.Cu) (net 13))
 (segment (start 175.736 83.28) (end 175.704 83.312) (width 0.25) (layer B.Cu) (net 13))
 (segment (start 175.704 83.312) (end 175.598668 83.312) (width 0.25) (layer B.Cu) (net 13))
 (segment (start 175.704 83.312) (end 173.736 83.312) (width 0.25) (layer B.Cu) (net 13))
 (segment (start 173.736 83.312) (end 173.736 81.449332) (width 0.25) (layer B.Cu) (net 13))
 (segment (start 172.746051 81.449332) (end 166.975 81.449332) (width 0.25) (layer B.Cu) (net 13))
 (segment (start 173.736 81.449332) (end 172.746051 81.449332) (width 0.25) (layer B.Cu) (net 13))
 (segment (start 132.588 71.628) (end 128.016 71.628) (width 0.25) (layer B.Cu) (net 13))
 (segment (start 132.588 73.152) (end 132.588 71.628) (width 0.25) (layer B.Cu) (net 13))
 (segment (start 150.876 73.152) (end 136.652 73.152) (width 0.25) (layer B.Cu) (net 13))
 (segment (start 166.975 81.449332) (end 166.975 82.149332) (width 0.25) (layer B.Cu) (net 13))
 (segment (start 167.132 82.306332) (end 167.132 84.328) (width 0.25) (layer B.Cu) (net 13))
 (segment (start 167.132 84.328) (end 150.876 84.328) (width 0.25) (layer B.Cu) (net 13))
 (segment (start 166.975 82.149332) (end 167.132 82.306332) (width 0.25) (layer B.Cu) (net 13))
 (segment (start 150.876 84.328) (end 150.876 73.152) (width 0.25) (layer B.Cu) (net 13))
 (segment (start 136.652 73.152) (end 132.588 73.152) (width 0.25) (layer B.Cu) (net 13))
 (via (at 136.652 73.152) (size 0.8) (drill 0.4) (layers F.Cu B.Cu) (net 13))
 (segment (start 136.652 73.152) (end 136.652 79.756) (width 0.25) (layer F.Cu) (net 13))
 (segment (start 136.652 79.756) (end 147.828 79.756) (width 0.25) (layer F.Cu) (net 13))
 (segment (start 147.828 79.756) (end 147.828 91.948) (width 0.25) (layer F.Cu) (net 13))
 (segment (start 147.828 91.948) (end 147.828 91.948) (width 0.25) (layer F.Cu) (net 13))
 (via (at 147.828 91.948) (size 0.8) (drill 0.4) (layers F.Cu B.Cu) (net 13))
 (segment (start 147.828 91.948) (end 141.224 91.948) (width 0.25) (layer B.Cu) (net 13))
 (segment (start 141.224 91.948) (end 141.224 91.948) (width 0.25) (layer B.Cu) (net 13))
 (via (at 141.224 91.948) (size 0.8) (drill 0.4) (layers F.Cu B.Cu) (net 13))
 (segment (start 141.224 87.959) (end 141.067 87.802) (width 0.25) (layer F.Cu) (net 13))
 (segment (start 141.224 91.948) (end 141.224 87.959) (width 0.25) (layer F.Cu) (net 13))
 (segment (start 175.736 87.460665) (end 175.736 89.884) (width 0.25) (layer B.Cu) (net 14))
 (segment (start 175.736 89.884) (end 175.704 89.916) (width 0.25) (layer B.Cu) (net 14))
 (segment (start 175.704 89.916) (end 173.736 89.916) (width 0.25) (layer B.Cu) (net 14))
 (segment (start 173.736 89.916) (end 173.736 87.460665) (width 0.25) (layer B.Cu) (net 14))
 (segment (start 172.746051 87.460665) (end 166.975 87.460665) (width 0.25) (layer B.Cu) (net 14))
 (segment (start 173.736 87.460665) (end 172.746051 87.460665) (width 0.25) (layer B.Cu) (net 14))
 (segment (start 166.975 87.460665) (end 166.975 90.267) (width 0.25) (layer B.Cu) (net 14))
 (segment (start 166.975 90.267) (end 166.818 90.424) (width 0.25) (layer B.Cu) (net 14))
 (segment (start 166.818 90.424) (end 148.844 90.424) (width 0.25) (layer B.Cu) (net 14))
 (segment (start 148.844 90.424) (end 148.844 74.676) (width 0.25) (layer B.Cu) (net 14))
 (segment (start 148.336 74.168) (end 128.016 74.168) (width 0.25) (layer B.Cu) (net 14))
 (segment (start 148.844 74.676) (end 148.336 74.168) (width 0.25) (layer B.Cu) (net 14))
 (segment (start 148.844 90.424) (end 148.844 92.964) (width 0.25) (layer B.Cu) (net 14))
 (segment (start 148.844 92.964) (end 142.24 92.964) (width 0.25) (layer B.Cu) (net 14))
 (segment (start 142.24 92.964) (end 142.24 92.964) (width 0.25) (layer B.Cu) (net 14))
 (via (at 142.24 92.964) (size 0.8) (drill 0.4) (layers F.Cu B.Cu) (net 14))
 (segment (start 142.24 87.879) (end 142.317 87.802) (width 0.25) (layer F.Cu) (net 14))
 (segment (start 142.24 92.964) (end 142.24 87.879) (width 0.25) (layer F.Cu) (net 14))
 (segment (start 175.736 94.461949) (end 175.768 94.493949) (width 0.25) (layer B.Cu) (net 15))
 (segment (start 175.736 93.472) (end 175.736 94.461949) (width 0.25) (layer B.Cu) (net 15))
 (segment (start 175.768 94.493949) (end 175.768 96.012) (width 0.25) (layer B.Cu) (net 15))
 (segment (start 175.768 96.012) (end 173.736 96.012) (width 0.25) (layer B.Cu) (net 15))
 (segment (start 173.736 96.012) (end 173.736 93.472) (width 0.25) (layer B.Cu) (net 15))
 (segment (start 173.736 93.472) (end 167.64 93.472) (width 0.25) (layer B.Cu) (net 15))
 (segment (start 167.64 93.472) (end 166.975 93.472) (width 0.25) (layer B.Cu) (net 15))
 (segment (start 128.016 76.708) (end 128.016 97.536) (width 0.25) (layer B.Cu) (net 15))
 (segment (start 128.016 97.536) (end 143.764 97.536) (width 0.25) (layer B.Cu) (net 15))
 (segment (start 167.132 97.536) (end 167.132 96.012) (width 0.25) (layer B.Cu) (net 15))
 (segment (start 166.975 95.855) (end 166.975 93.472) (width 0.25) (layer B.Cu) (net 15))
 (segment (start 167.132 96.012) (end 166.975 95.855) (width 0.25) (layer B.Cu) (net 15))
 (segment (start 143.764 97.536) (end 167.132 97.536) (width 0.25) (layer B.Cu) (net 15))
 (via (at 143.764 97.536) (size 0.8) (drill 0.4) (layers F.Cu B.Cu) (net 15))
 (segment (start 143.764 87.999) (end 143.567 87.802) (width 0.25) (layer F.Cu) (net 15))
 (segment (start 143.764 97.536) (end 143.764 87.999) (width 0.25) (layer F.Cu) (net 15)))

